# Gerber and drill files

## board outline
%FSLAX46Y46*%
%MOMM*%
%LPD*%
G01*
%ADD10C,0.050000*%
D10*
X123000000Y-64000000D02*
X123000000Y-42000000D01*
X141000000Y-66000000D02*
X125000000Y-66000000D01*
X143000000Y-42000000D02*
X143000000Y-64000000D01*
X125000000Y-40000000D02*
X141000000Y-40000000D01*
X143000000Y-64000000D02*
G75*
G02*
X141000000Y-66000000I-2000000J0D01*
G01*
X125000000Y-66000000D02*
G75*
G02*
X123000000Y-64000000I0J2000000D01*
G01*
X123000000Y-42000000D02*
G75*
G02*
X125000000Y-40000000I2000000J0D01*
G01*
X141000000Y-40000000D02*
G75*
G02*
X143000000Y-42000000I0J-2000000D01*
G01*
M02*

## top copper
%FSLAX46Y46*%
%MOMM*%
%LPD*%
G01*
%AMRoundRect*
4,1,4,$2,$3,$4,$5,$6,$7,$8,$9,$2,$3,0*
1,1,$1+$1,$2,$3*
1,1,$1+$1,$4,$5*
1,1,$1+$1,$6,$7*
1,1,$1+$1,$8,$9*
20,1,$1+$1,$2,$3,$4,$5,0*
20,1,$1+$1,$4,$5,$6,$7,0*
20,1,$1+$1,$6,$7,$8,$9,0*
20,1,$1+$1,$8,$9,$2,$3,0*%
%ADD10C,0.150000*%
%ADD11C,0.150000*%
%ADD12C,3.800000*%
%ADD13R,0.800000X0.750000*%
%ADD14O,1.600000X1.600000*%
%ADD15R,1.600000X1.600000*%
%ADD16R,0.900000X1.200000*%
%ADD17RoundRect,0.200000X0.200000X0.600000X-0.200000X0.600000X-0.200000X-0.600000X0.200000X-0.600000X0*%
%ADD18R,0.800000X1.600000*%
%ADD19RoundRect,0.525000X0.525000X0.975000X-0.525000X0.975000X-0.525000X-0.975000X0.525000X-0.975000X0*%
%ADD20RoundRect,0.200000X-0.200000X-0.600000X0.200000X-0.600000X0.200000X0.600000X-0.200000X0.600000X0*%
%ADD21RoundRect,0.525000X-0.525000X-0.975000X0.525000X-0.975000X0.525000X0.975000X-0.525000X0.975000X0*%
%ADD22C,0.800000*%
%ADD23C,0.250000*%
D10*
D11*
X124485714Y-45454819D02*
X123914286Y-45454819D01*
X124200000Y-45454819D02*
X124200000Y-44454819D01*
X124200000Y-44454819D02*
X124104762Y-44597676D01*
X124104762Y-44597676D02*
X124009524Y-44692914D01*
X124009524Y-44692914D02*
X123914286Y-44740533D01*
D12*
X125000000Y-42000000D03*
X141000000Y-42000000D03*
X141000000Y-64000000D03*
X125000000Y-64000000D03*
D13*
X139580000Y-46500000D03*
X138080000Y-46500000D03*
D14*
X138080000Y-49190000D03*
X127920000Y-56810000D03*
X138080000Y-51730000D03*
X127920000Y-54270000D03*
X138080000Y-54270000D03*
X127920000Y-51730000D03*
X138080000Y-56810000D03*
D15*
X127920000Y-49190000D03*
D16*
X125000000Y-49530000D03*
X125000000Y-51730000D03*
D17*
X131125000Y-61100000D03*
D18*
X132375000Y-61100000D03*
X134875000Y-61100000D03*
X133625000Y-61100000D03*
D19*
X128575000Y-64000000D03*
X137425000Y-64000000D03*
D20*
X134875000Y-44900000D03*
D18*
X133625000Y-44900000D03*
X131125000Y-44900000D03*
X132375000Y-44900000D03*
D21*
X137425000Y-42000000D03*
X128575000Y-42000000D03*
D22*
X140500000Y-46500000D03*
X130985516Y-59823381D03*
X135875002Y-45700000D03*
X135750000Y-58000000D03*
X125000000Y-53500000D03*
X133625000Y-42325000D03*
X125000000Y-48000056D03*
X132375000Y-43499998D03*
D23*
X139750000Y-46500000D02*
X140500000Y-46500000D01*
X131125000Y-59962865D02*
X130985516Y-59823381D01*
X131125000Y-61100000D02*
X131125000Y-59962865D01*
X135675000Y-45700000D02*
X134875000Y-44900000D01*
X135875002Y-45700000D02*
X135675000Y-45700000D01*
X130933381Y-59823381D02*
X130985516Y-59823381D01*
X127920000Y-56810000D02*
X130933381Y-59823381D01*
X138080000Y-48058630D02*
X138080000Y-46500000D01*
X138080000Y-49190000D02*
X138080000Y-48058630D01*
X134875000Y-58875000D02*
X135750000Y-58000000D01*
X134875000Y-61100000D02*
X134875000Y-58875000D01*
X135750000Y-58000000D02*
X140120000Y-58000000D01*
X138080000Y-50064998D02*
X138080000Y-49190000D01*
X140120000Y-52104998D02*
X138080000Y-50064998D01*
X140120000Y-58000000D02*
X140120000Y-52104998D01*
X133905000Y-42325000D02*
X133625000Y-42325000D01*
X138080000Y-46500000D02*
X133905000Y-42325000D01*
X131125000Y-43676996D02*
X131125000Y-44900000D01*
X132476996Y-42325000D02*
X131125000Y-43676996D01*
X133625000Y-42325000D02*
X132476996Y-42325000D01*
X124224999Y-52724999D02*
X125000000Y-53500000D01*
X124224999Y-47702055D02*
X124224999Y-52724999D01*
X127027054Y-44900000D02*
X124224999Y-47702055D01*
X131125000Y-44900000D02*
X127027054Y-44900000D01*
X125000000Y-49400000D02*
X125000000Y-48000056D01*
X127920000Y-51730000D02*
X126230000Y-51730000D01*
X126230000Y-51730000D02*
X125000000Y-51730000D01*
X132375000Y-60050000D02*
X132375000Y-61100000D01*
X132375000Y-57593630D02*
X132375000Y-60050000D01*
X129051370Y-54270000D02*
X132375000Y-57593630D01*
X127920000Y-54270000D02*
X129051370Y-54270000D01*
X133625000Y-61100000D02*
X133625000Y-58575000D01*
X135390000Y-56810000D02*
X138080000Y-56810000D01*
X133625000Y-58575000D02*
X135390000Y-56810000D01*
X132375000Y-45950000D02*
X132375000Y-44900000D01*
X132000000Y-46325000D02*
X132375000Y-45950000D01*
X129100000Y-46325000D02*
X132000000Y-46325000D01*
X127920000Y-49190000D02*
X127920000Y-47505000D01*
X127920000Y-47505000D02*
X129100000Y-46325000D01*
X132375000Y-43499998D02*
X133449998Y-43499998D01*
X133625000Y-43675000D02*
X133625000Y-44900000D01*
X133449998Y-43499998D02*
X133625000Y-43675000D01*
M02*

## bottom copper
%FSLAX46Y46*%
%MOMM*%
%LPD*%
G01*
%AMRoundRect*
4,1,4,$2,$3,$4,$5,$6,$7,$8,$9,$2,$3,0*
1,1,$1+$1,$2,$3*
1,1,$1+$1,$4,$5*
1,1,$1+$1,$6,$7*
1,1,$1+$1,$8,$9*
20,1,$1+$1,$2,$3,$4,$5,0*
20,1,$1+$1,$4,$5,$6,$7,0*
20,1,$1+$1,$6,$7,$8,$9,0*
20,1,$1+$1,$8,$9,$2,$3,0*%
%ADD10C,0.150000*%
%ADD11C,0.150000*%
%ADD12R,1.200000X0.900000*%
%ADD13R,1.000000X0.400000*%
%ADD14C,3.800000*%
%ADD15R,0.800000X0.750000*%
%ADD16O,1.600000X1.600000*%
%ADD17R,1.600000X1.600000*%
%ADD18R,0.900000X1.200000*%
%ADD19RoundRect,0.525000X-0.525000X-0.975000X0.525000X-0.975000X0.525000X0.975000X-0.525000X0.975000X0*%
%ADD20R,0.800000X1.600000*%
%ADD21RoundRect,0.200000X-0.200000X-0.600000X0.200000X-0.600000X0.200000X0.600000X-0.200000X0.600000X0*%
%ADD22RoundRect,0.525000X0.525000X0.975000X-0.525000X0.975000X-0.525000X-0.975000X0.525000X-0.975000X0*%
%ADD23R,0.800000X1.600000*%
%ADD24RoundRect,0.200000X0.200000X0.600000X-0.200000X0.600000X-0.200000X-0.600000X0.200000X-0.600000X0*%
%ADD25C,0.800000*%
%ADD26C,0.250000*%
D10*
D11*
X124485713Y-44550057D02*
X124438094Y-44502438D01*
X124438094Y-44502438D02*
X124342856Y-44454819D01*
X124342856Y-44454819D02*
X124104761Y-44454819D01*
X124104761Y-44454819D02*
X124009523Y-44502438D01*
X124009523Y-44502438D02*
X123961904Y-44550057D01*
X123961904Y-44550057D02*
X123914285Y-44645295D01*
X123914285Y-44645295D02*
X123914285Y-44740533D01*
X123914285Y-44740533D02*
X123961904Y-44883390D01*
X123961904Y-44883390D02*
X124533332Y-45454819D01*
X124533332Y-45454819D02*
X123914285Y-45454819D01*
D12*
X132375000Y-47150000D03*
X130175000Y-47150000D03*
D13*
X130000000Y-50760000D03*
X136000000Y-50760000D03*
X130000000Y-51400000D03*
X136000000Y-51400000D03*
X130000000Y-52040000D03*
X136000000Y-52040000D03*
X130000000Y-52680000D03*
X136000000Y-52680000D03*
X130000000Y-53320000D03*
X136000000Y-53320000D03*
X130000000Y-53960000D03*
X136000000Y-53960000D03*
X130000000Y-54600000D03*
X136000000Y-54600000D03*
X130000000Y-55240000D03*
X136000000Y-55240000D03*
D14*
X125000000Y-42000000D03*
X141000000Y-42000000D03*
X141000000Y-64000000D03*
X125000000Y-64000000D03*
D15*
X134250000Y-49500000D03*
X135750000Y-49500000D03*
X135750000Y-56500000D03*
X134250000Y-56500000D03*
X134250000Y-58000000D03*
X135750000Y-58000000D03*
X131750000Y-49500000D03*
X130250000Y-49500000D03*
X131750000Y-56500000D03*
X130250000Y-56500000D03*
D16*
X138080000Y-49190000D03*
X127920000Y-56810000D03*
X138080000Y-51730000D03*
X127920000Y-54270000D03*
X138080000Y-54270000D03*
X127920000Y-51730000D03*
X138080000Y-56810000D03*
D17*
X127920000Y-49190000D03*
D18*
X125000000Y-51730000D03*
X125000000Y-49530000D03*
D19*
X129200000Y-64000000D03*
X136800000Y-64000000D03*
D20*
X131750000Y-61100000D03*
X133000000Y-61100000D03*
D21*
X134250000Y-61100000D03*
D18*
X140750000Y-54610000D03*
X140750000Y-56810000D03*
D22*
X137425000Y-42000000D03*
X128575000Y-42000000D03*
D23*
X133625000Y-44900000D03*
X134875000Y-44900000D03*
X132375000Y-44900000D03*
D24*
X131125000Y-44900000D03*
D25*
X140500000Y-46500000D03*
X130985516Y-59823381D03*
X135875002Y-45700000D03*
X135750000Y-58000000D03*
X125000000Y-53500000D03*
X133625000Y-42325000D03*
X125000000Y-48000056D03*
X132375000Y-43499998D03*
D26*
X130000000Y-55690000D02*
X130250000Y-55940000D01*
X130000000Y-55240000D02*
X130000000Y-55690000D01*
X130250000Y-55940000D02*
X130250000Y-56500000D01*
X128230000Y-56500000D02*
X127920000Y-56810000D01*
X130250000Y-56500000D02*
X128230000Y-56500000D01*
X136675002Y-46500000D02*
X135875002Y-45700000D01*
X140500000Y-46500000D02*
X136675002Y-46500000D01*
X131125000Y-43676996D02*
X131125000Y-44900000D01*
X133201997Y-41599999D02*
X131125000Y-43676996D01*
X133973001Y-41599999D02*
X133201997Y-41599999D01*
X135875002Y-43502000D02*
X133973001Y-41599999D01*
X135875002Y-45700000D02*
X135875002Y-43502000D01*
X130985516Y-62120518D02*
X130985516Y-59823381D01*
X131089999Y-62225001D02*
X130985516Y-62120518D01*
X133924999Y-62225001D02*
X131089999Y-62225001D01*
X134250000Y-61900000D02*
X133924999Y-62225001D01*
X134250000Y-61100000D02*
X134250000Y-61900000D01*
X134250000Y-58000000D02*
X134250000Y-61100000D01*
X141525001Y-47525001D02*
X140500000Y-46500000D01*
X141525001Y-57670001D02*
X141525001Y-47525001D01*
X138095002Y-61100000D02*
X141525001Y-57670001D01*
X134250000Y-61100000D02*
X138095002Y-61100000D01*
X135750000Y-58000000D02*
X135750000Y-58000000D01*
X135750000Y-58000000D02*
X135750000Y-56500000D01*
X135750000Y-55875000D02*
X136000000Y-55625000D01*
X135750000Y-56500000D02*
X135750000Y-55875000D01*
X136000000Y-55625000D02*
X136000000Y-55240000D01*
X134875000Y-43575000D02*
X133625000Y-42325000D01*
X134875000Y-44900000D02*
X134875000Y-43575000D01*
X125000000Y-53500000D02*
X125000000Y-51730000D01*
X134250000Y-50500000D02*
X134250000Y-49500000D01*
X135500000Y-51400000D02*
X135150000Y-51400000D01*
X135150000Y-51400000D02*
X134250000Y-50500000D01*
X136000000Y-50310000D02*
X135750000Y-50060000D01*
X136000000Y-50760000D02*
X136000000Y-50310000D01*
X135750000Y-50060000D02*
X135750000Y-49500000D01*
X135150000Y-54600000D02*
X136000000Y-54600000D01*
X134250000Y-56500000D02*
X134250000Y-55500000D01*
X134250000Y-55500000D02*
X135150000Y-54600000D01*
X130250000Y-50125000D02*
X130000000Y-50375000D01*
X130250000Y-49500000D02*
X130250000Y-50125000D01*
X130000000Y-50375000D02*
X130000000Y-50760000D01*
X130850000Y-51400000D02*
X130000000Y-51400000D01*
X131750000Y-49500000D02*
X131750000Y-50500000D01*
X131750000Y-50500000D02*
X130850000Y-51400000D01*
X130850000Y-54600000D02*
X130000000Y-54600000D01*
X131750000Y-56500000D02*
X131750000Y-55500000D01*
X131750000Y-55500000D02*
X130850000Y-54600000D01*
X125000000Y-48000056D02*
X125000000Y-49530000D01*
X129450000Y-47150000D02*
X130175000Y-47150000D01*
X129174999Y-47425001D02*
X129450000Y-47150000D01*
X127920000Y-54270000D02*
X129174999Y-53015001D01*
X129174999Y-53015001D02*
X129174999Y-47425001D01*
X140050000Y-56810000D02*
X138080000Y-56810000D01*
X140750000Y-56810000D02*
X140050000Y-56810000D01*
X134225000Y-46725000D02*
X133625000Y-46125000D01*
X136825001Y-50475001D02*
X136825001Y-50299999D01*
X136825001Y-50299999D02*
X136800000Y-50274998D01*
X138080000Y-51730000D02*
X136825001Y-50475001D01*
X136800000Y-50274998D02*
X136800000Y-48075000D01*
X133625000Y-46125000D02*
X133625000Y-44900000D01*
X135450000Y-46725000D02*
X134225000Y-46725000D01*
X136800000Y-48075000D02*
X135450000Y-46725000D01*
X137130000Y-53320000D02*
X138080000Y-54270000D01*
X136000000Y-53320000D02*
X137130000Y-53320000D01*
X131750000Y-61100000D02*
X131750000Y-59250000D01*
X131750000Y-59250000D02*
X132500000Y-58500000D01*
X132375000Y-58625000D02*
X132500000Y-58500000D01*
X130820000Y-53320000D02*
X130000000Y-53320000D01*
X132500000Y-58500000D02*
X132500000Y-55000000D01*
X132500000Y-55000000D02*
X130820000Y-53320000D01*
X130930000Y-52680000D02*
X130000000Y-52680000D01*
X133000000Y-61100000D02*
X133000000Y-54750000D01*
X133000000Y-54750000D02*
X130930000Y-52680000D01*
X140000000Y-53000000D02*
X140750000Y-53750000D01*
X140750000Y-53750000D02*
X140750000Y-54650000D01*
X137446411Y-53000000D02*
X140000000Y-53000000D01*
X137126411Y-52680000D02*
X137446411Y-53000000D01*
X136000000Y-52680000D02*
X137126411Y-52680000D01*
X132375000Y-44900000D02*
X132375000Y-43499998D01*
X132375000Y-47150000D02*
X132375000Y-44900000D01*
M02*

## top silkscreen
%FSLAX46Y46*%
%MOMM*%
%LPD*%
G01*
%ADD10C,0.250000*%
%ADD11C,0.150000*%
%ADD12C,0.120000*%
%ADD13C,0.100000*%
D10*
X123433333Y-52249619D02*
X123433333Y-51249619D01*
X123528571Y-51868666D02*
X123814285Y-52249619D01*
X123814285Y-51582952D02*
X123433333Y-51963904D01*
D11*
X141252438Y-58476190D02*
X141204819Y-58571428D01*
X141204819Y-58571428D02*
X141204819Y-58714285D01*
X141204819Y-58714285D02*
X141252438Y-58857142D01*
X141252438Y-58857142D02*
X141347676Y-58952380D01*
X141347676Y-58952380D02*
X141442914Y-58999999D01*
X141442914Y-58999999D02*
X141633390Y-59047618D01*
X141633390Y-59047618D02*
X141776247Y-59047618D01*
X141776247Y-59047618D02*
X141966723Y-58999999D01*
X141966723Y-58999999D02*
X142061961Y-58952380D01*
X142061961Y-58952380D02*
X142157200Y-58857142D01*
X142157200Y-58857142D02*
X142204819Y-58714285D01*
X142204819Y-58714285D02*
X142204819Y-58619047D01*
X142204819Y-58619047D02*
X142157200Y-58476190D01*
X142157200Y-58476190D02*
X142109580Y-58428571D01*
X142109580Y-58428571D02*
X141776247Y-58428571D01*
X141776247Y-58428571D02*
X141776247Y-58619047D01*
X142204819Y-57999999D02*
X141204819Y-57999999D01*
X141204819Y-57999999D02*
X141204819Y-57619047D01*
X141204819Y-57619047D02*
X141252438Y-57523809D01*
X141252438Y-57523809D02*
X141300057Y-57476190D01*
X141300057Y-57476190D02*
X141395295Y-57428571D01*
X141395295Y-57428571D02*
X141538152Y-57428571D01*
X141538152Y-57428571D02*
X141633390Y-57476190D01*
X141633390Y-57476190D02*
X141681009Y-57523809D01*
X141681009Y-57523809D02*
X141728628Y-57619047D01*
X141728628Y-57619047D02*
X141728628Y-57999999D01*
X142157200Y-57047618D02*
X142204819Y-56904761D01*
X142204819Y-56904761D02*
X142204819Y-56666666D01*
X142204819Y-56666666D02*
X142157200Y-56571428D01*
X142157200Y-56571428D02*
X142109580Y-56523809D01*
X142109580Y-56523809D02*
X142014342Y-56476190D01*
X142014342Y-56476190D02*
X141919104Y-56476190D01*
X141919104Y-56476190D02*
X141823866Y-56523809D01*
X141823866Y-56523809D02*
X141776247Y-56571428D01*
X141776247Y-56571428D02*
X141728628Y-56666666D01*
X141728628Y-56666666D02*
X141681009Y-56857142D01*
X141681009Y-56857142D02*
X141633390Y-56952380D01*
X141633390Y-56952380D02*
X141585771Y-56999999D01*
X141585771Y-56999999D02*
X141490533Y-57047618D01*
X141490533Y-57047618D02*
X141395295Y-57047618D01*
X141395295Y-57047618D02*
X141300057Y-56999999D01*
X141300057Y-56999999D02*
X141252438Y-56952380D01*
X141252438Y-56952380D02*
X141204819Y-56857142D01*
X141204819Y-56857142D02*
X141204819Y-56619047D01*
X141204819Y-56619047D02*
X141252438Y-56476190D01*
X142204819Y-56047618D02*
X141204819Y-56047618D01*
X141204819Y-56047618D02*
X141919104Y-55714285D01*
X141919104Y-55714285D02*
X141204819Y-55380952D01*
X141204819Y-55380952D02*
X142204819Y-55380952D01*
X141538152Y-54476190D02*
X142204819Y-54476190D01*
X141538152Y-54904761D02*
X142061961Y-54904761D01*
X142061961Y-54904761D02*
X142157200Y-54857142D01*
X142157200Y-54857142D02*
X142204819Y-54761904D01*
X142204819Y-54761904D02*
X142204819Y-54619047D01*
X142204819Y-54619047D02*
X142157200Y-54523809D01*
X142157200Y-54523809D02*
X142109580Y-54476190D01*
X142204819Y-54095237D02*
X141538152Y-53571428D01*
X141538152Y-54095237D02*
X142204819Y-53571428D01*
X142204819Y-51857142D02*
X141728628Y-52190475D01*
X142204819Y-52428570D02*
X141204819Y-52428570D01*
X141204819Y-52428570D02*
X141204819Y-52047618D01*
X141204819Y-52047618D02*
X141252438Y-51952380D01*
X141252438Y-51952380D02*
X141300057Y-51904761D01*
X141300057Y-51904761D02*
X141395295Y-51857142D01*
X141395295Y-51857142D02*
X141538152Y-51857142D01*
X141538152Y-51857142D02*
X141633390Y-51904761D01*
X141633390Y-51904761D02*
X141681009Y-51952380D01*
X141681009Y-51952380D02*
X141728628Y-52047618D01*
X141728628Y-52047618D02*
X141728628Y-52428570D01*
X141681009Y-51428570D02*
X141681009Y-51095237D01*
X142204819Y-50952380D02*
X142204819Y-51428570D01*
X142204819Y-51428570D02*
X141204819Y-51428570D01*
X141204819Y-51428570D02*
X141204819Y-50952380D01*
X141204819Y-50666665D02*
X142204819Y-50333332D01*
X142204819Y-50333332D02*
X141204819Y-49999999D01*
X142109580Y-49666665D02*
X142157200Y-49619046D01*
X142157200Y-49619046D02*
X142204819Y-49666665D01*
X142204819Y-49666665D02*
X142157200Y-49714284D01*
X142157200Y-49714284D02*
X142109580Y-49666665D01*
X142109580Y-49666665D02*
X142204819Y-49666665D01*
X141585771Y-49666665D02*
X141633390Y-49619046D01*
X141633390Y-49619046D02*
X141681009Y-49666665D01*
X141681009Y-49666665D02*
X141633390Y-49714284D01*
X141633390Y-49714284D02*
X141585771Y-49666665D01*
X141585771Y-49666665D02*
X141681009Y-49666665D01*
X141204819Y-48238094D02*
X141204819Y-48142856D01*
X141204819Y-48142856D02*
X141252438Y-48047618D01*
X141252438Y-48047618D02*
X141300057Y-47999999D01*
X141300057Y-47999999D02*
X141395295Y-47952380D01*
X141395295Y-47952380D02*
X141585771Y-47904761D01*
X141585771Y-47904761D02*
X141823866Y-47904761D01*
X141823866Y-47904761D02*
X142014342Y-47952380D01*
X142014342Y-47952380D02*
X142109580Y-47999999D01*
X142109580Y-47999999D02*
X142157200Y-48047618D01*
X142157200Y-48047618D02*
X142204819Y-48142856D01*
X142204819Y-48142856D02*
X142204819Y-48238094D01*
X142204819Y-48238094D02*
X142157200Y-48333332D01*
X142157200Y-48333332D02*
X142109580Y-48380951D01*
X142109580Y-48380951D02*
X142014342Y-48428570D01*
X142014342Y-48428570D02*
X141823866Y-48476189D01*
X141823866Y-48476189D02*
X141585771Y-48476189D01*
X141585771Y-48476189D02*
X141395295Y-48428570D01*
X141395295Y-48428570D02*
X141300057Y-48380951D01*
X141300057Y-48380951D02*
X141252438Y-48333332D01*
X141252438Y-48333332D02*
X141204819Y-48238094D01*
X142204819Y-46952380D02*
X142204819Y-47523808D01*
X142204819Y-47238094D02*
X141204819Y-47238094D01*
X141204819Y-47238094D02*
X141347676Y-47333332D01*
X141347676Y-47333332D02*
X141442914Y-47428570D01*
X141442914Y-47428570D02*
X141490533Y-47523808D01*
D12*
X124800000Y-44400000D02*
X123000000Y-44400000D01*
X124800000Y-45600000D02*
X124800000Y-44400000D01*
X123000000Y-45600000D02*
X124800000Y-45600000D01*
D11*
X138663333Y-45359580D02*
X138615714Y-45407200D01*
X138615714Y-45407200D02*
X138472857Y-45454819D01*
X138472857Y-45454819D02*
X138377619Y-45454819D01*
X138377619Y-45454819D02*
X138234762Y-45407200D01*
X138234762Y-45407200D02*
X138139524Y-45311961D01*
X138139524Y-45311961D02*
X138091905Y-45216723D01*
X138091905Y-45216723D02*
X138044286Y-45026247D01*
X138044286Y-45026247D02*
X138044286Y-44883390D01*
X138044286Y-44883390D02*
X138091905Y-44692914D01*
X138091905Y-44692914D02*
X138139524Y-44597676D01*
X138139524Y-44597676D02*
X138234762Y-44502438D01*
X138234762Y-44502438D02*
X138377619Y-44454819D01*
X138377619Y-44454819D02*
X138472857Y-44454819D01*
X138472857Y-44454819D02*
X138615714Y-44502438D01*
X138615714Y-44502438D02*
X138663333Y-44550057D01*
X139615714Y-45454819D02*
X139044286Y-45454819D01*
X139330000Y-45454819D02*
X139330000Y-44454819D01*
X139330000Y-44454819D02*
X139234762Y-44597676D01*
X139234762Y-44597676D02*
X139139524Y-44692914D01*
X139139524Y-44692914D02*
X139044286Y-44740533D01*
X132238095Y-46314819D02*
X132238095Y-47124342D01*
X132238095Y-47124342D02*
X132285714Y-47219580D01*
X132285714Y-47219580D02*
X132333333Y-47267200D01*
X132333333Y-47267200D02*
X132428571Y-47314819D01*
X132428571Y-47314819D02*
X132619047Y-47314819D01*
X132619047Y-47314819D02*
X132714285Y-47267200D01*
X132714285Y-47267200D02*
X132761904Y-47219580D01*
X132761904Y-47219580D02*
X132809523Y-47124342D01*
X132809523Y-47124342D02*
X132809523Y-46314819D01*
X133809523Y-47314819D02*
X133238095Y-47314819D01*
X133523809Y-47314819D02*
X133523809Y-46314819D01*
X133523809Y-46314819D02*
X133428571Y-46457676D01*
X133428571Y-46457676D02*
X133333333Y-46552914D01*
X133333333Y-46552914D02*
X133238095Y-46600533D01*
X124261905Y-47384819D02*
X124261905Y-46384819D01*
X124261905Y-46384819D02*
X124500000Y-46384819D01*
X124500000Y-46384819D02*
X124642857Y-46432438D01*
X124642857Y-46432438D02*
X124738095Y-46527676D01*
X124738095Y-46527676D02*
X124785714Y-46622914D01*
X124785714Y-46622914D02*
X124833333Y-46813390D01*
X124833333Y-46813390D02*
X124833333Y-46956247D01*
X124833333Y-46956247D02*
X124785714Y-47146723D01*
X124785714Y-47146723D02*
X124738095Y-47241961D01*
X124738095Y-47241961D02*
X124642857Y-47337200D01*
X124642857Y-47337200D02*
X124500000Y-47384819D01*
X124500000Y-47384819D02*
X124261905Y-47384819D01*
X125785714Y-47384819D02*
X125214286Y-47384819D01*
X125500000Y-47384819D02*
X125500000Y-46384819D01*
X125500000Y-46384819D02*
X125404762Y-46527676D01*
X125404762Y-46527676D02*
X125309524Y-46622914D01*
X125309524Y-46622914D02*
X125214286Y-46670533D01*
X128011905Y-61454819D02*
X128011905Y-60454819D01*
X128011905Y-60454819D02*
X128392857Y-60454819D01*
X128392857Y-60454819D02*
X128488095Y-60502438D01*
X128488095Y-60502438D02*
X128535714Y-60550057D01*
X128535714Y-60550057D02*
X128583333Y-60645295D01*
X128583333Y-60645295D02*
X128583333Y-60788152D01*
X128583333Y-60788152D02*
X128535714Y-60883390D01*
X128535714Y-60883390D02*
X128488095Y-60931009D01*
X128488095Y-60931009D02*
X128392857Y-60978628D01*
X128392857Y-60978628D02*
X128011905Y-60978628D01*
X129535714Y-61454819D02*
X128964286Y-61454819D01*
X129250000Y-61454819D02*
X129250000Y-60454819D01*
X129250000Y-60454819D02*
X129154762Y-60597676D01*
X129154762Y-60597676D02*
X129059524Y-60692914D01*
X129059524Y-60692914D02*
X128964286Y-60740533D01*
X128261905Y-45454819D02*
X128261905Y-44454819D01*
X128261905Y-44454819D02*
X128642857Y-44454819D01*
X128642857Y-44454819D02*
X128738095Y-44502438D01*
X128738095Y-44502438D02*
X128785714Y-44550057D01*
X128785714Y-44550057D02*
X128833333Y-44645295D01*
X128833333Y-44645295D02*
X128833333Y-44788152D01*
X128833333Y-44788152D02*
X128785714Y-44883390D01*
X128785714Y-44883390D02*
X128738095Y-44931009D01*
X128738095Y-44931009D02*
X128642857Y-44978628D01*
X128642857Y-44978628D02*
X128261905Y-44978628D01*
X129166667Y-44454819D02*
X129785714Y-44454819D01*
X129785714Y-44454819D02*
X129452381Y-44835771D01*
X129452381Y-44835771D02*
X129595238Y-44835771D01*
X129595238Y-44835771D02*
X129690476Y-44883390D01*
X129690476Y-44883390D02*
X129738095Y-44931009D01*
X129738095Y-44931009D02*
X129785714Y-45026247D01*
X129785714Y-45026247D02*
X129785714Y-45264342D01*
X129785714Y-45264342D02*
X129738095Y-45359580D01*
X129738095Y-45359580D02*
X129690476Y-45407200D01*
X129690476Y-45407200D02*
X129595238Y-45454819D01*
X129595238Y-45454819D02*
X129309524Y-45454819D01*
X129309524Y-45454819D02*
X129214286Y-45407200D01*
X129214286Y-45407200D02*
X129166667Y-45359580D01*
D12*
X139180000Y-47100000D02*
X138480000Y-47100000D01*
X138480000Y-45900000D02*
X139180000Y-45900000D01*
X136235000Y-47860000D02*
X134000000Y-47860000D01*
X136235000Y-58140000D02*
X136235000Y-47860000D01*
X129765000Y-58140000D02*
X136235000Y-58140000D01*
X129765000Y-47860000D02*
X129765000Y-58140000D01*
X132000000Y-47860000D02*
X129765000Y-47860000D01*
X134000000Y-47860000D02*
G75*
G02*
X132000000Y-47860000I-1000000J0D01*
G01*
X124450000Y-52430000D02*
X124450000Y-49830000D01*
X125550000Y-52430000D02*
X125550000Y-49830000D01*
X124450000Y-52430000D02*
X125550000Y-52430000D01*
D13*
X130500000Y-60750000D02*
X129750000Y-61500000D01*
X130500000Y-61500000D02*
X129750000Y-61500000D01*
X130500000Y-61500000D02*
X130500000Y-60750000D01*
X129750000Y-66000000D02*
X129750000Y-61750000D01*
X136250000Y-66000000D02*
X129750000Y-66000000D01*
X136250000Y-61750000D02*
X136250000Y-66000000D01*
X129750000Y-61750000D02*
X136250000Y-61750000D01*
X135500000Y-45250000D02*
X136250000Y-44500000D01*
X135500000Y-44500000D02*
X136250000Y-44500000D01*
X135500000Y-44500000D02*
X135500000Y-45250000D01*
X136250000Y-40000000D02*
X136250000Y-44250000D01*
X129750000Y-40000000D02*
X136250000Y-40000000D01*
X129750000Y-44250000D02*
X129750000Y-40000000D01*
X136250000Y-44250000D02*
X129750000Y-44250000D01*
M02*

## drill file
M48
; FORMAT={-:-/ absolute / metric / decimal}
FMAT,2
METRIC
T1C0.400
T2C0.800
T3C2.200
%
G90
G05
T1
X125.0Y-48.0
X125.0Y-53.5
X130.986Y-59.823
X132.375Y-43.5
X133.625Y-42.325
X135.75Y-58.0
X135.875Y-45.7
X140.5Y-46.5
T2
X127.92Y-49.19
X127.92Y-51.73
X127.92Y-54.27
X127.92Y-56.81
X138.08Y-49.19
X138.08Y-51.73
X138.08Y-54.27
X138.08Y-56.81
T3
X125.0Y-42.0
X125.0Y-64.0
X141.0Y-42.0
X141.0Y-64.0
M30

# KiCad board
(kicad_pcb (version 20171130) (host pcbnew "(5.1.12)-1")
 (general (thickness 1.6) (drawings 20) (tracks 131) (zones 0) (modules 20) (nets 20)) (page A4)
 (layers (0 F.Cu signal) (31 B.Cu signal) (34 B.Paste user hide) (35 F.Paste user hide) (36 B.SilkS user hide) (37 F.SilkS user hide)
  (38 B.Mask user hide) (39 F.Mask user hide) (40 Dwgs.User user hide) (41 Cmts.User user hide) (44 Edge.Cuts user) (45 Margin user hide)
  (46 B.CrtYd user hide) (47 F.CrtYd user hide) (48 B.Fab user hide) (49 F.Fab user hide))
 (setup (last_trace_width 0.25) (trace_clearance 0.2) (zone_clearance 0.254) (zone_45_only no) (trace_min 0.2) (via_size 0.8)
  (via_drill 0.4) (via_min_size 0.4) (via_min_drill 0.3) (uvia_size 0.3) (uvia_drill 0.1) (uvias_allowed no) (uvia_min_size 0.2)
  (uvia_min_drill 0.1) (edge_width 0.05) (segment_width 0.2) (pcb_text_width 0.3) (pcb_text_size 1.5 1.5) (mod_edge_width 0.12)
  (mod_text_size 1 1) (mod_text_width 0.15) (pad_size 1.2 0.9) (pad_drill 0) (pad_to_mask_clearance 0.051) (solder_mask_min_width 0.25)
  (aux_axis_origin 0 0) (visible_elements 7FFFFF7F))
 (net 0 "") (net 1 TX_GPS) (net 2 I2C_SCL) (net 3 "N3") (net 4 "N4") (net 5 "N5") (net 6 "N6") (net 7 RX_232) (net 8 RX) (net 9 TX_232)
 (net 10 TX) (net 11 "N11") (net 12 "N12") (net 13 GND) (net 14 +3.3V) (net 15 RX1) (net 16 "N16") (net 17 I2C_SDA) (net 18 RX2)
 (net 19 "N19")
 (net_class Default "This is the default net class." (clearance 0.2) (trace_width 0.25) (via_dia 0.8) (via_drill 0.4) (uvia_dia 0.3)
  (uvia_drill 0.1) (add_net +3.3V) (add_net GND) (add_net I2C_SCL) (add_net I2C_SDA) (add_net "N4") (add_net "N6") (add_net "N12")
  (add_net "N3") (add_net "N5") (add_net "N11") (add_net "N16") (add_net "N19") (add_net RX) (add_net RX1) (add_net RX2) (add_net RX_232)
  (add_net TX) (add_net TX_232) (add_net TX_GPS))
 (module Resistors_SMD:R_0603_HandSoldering (layer B.Cu) (at 131.275 47.15 180)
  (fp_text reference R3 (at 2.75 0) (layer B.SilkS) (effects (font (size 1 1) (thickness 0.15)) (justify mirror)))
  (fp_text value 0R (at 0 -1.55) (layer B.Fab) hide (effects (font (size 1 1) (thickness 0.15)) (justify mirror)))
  (pad 1 smd rect (at -1.1 0 180) (size 1.2 0.9) (layers B.Cu B.Paste B.Mask) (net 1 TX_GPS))
  (pad 2 smd rect (at 1.1 0 180) (size 1.2 0.9) (layers B.Cu B.Paste B.Mask) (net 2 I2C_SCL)))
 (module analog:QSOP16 (layer B.Cu) (at 133 53 270) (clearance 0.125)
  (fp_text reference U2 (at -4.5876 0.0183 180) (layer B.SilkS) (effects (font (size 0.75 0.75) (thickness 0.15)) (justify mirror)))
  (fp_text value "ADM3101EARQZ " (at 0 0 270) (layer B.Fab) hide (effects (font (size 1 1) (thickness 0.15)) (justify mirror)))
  (pad 16 smd rect (at -2.24 3 270) (size 0.4 1) (layers B.Cu B.Paste B.Mask) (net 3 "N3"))
  (pad 1 smd rect (at -2.24 -3 270) (size 0.4 1) (layers B.Cu B.Paste B.Mask) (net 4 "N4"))
  (pad 15 smd rect (at -1.6 3 270) (size 0.4 1) (layers B.Cu B.Paste B.Mask) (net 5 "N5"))
  (pad 2 smd rect (at -1.6 -3 270) (size 0.4 1) (layers B.Cu B.Paste B.Mask) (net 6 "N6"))
  (pad 14 smd rect (at -0.96 3 270) (size 0.4 1) (layers B.Cu B.Paste B.Mask))
  (pad 3 smd rect (at -0.96 -3 270) (size 0.4 1) (layers B.Cu B.Paste B.Mask))
  (pad 13 smd rect (at -0.32 3 270) (size 0.4 1) (layers B.Cu B.Paste B.Mask) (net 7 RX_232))
  (pad 4 smd rect (at -0.32 -3 270) (size 0.4 1) (layers B.Cu B.Paste B.Mask) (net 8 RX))
  (pad 12 smd rect (at 0.32 3 270) (size 0.4 1) (layers B.Cu B.Paste B.Mask) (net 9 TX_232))
  (pad 5 smd rect (at 0.32 -3 270) (size 0.4 1) (layers B.Cu B.Paste B.Mask) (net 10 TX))
  (pad 11 smd rect (at 0.96 3 270) (size 0.4 1) (layers B.Cu B.Paste B.Mask))
  (pad 6 smd rect (at 0.96 -3 270) (size 0.4 1) (layers B.Cu B.Paste B.Mask))
  (pad 10 smd rect (at 1.6 3 270) (size 0.4 1) (layers B.Cu B.Paste B.Mask) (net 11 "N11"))
  (pad 7 smd rect (at 1.6 -3 270) (size 0.4 1) (layers B.Cu B.Paste B.Mask) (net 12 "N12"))
  (pad 9 smd rect (at 2.24 3 270) (size 0.4 1) (layers B.Cu B.Paste B.Mask) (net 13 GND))
  (pad 8 smd rect (at 2.24 -3 270) (size 0.4 1) (layers B.Cu B.Paste B.Mask) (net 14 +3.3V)))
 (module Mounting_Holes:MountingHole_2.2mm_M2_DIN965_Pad (layer F.Cu) (at 125 42)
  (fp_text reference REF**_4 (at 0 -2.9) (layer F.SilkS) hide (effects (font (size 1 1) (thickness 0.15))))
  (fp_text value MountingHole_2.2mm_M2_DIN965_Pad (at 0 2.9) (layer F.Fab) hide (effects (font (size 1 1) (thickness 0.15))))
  (pad 1 thru_hole circle (at 0 0) (size 3.8 3.8) (drill 2.2) (layers *.Cu *.Mask)))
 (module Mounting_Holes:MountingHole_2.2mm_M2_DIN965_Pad (layer F.Cu) (at 141 42)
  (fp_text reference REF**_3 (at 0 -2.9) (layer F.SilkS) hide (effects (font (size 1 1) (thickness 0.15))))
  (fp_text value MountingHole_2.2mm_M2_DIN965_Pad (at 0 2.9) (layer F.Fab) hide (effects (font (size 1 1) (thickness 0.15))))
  (pad 1 thru_hole circle (at 0 0) (size 3.8 3.8) (drill 2.2) (layers *.Cu *.Mask)))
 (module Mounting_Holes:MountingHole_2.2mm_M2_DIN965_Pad (layer F.Cu) (at 141 64)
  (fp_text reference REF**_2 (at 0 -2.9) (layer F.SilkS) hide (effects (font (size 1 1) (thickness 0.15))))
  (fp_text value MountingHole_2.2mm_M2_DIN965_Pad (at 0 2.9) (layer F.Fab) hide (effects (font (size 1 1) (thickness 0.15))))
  (pad 1 thru_hole circle (at 0 0) (size 3.8 3.8) (drill 2.2) (layers *.Cu *.Mask)))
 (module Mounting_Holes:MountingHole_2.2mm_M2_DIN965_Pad (layer F.Cu) (at 125 64)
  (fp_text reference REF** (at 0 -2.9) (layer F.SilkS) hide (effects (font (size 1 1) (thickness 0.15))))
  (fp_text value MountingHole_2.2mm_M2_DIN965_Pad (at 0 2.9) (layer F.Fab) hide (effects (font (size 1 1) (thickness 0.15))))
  (pad 1 thru_hole circle (at 0 0) (size 3.8 3.8) (drill 2.2) (layers *.Cu *.Mask)))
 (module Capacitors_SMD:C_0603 (layer F.Cu) (at 138.83 46.5)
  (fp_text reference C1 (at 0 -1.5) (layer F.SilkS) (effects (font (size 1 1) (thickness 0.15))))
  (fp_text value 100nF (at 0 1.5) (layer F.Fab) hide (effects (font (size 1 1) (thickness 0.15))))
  (fp_line (start 0.35 0.6) (end -0.35 0.6) (layer F.SilkS) (width 0.12))
  (fp_line (start -0.35 -0.6) (end 0.35 -0.6) (layer F.SilkS) (width 0.12))
  (pad 2 smd rect (at 0.75 0) (size 0.8 0.75) (layers F.Cu F.Paste F.Mask) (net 13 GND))
  (pad 1 smd rect (at -0.75 0) (size 0.8 0.75) (layers F.Cu F.Paste F.Mask) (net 14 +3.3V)))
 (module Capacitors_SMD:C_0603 (layer B.Cu) (at 135 49.5 180)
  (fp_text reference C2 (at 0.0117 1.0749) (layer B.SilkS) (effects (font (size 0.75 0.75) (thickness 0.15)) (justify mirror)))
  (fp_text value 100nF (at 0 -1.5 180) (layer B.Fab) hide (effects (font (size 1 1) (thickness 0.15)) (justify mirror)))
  (pad 2 smd rect (at 0.75 0 180) (size 0.8 0.75) (layers B.Cu B.Paste B.Mask) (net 6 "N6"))
  (pad 1 smd rect (at -0.75 0 180) (size 0.8 0.75) (layers B.Cu B.Paste B.Mask) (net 4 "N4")))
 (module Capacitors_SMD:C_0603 (layer B.Cu) (at 135 56.5)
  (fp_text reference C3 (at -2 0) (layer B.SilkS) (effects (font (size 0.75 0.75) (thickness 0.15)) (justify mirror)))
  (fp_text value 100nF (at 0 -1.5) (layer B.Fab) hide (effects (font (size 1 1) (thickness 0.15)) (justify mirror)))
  (pad 2 smd rect (at 0.75 0) (size 0.8 0.75) (layers B.Cu B.Paste B.Mask) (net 14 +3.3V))
  (pad 1 smd rect (at -0.75 0) (size 0.8 0.75) (layers B.Cu B.Paste B.Mask) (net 12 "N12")))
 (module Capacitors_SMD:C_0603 (layer B.Cu) (at 135 58 180)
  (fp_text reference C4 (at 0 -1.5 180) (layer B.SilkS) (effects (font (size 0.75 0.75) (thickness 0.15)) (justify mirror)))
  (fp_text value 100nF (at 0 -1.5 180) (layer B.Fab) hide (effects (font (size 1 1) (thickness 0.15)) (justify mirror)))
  (pad 2 smd rect (at 0.75 0 180) (size 0.8 0.75) (layers B.Cu B.Paste B.Mask) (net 13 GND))
  (pad 1 smd rect (at -0.75 0 180) (size 0.8 0.75) (layers B.Cu B.Paste B.Mask) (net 14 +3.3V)))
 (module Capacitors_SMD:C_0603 (layer B.Cu) (at 131 49.5)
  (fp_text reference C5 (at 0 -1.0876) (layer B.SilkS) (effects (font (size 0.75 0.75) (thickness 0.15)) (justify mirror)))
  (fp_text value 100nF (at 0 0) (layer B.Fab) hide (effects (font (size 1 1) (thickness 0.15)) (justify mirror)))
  (pad 2 smd rect (at 0.75 0) (size 0.8 0.75) (layers B.Cu B.Paste B.Mask) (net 5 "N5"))
  (pad 1 smd rect (at -0.75 0) (size 0.8 0.75) (layers B.Cu B.Paste B.Mask) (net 3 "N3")))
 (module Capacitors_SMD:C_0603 (layer B.Cu) (at 131 56.5)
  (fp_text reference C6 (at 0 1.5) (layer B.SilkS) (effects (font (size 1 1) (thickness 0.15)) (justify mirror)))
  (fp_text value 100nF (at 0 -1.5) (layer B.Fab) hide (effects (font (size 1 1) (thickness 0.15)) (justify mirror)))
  (pad 2 smd rect (at 0.75 0) (size 0.8 0.75) (layers B.Cu B.Paste B.Mask) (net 11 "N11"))
  (pad 1 smd rect (at -0.75 0) (size 0.8 0.75) (layers B.Cu B.Paste B.Mask) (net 13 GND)))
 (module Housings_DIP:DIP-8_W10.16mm (layer F.Cu) (at 133 53)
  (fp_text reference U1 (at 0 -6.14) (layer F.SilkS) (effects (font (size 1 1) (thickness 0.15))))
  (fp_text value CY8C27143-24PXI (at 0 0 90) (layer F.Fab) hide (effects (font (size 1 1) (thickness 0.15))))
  (fp_line (start 3.235 -5.14) (end 1 -5.14) (layer F.SilkS) (width 0.12))
  (fp_line (start 3.235 5.14) (end 3.235 -5.14) (layer F.SilkS) (width 0.12))
  (fp_line (start -3.235 5.14) (end 3.235 5.14) (layer F.SilkS) (width 0.12))
  (fp_line (start -3.235 -5.14) (end -3.235 5.14) (layer F.SilkS) (width 0.12))
  (fp_line (start -1 -5.14) (end -3.235 -5.14) (layer F.SilkS) (width 0.12))
  (fp_arc (start 0 -5.14) (end -1 -5.14) (angle -180) (layer F.SilkS) (width 0.12))
  (pad 8 thru_hole oval (at 5.08 -3.81) (size 1.6 1.6) (drill 0.8) (layers *.Cu *.Mask) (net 14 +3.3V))
  (pad 4 thru_hole oval (at -5.08 3.81) (size 1.6 1.6) (drill 0.8) (layers *.Cu *.Mask) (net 13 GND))
  (pad 7 thru_hole oval (at 5.08 -1.27) (size 1.6 1.6) (drill 0.8) (layers *.Cu *.Mask) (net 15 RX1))
  (pad 3 thru_hole oval (at -5.08 1.27) (size 1.6 1.6) (drill 0.8) (layers *.Cu *.Mask) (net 2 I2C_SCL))
  (pad 6 thru_hole oval (at 5.08 1.27) (size 1.6 1.6) (drill 0.8) (layers *.Cu *.Mask) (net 10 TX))
  (pad 2 thru_hole oval (at -5.08 -1.27) (size 1.6 1.6) (drill 0.8) (layers *.Cu *.Mask) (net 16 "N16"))
  (pad 5 thru_hole oval (at 5.08 3.81) (size 1.6 1.6) (drill 0.8) (layers *.Cu *.Mask) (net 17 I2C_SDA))
  (pad 1 thru_hole rect (at -5.08 -3.81) (size 1.6 1.6) (drill 0.8) (layers *.Cu *.Mask) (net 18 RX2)))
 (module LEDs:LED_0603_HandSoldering (layer F.Cu) (at 125 50.63 90)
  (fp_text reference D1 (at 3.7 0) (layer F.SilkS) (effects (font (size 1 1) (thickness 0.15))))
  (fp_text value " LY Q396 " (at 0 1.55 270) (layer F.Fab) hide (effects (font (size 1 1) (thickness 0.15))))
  (fp_line (start -1.8 -0.55) (end 0.8 -0.55) (layer F.SilkS) (width 0.12))
  (fp_line (start -1.8 0.55) (end 0.8 0.55) (layer F.SilkS) (width 0.12))
  (fp_line (start -1.8 -0.55) (end -1.8 0.55) (layer F.SilkS) (width 0.12))
  (pad 2 smd rect (at 1.1 0 90) (size 1.2 0.9) (layers F.Cu F.Paste F.Mask) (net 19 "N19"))
  (pad 1 smd rect (at -1.1 0 90) (size 1.2 0.9) (layers F.Cu F.Paste F.Mask) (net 16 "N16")))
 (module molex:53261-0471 (layer F.Cu) (at 133 64 180) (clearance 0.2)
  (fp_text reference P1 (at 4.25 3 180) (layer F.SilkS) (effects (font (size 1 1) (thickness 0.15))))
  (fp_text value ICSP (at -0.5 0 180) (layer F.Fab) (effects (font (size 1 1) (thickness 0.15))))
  (fp_line (start 2.5 3.25) (end 3.25 2.5) (layer F.SilkS) (width 0.1))
  (fp_line (start 2.5 2.5) (end 3.25 2.5) (layer F.SilkS) (width 0.1))
  (fp_line (start 2.5 2.5) (end 2.5 3.25) (layer F.SilkS) (width 0.1))
  (fp_line (start 3.25 -2) (end 3.25 2.25) (layer F.SilkS) (width 0.1))
  (fp_line (start -3.25 -2) (end 3.25 -2) (layer F.SilkS) (width 0.1))
  (fp_line (start -3.25 2.25) (end -3.25 -2) (layer F.SilkS) (width 0.1))
  (fp_line (start 3.25 2.25) (end -3.25 2.25) (layer F.SilkS) (width 0.1))
  (pad 1 connect roundrect (at 1.875 2.9 180) (size 0.8 1.6) (layers F.Cu F.Mask) (roundrect_rratio 0.25) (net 13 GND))
  (pad 2 connect rect (at 0.625 2.9 180) (size 0.8 1.6) (layers F.Cu F.Mask) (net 2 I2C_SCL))
  (pad 4 connect rect (at -1.875 2.9 180) (size 0.8 1.6) (layers F.Cu F.Mask) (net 14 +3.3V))
  (pad 3 connect rect (at -0.625 2.9 180) (size 0.8 1.6) (layers F.Cu F.Mask) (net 17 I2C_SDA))
  (pad "" connect roundrect (at 4.425 0 180) (size 2.1 3) (layers F.Cu F.Mask) (roundrect_rratio 0.25))
  (pad "" connect roundrect (at -4.425 0 180) (size 2.1 3) (layers F.Cu F.Mask) (roundrect_rratio 0.25)))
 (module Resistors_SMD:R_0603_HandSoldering (layer B.Cu) (at 125 50.63 270)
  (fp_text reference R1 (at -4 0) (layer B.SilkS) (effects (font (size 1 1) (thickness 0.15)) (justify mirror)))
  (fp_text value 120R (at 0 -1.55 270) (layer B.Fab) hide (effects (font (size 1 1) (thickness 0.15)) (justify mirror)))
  (pad 2 smd rect (at 1.1 0 270) (size 1.2 0.9) (layers B.Cu B.Paste B.Mask) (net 14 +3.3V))
  (pad 1 smd rect (at -1.1 0 270) (size 1.2 0.9) (layers B.Cu B.Paste B.Mask) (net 19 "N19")))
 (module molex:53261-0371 (layer B.Cu) (at 133 64) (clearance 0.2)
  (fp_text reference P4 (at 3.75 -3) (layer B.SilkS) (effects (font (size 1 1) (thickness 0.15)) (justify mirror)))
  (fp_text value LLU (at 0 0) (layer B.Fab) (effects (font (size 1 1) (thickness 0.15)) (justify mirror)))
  (pad "" connect roundrect (at -3.8 0) (size 2.1 3) (layers B.Cu B.Mask) (roundrect_rratio 0.25))
  (pad "" connect roundrect (at 3.8 0) (size 2.1 3) (layers B.Cu B.Mask) (roundrect_rratio 0.25))
  (pad 3 smd rect (at -1.25 -2.9) (size 0.8 1.6) (layers B.Cu B.Paste B.Mask) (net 9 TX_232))
  (pad 2 smd rect (at 0 -2.9) (size 0.8 1.6) (layers B.Cu B.Paste B.Mask) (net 7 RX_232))
  (pad 1 smd roundrect (at 1.25 -2.9) (size 0.8 1.6) (layers B.Cu B.Paste B.Mask) (roundrect_rratio 0.25) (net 13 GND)))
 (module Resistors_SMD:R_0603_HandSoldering (layer B.Cu) (at 140.75 55.71 90)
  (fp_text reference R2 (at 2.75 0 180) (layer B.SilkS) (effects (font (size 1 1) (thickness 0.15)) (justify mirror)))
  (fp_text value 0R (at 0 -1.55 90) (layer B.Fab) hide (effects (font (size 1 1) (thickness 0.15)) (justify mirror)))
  (pad 2 smd rect (at 1.1 0 90) (size 1.2 0.9) (layers B.Cu B.Paste B.Mask) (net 8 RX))
  (pad 1 smd rect (at -1.1 0 90) (size 1.2 0.9) (layers B.Cu B.Paste B.Mask) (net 17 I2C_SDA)))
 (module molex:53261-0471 (layer B.Cu) (at 133 42 180) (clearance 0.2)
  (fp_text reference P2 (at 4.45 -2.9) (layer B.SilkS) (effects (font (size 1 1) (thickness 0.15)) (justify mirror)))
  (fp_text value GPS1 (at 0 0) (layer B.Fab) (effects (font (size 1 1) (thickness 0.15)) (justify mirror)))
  (pad "" connect roundrect (at -4.425 0 180) (size 2.1 3) (layers B.Cu B.Mask) (roundrect_rratio 0.25))
  (pad "" connect roundrect (at 4.425 0 180) (size 2.1 3) (layers B.Cu B.Mask) (roundrect_rratio 0.25))
  (pad 3 connect rect (at -0.625 -2.9 180) (size 0.8 1.6) (layers B.Cu B.Mask) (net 15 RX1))
  (pad 4 connect rect (at -1.875 -2.9 180) (size 0.8 1.6) (layers B.Cu B.Mask) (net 14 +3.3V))
  (pad 2 connect rect (at 0.625 -2.9 180) (size 0.8 1.6) (layers B.Cu B.Mask) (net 1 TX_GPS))
  (pad 1 connect roundrect (at 1.875 -2.9 180) (size 0.8 1.6) (layers B.Cu B.Mask) (roundrect_rratio 0.25) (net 13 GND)))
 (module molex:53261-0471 (layer F.Cu) (at 133 42) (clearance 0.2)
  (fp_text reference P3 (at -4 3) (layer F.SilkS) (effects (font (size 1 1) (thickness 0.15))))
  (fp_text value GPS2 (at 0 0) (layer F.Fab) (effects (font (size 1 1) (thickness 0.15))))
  (fp_line (start 2.5 3.25) (end 3.25 2.5) (layer F.SilkS) (width 0.1))
  (fp_line (start 2.5 2.5) (end 3.25 2.5) (layer F.SilkS) (width 0.1))
  (fp_line (start 2.5 2.5) (end 2.5 3.25) (layer F.SilkS) (width 0.1))
  (fp_line (start 3.25 -2) (end 3.25 2.25) (layer F.SilkS) (width 0.1))
  (fp_line (start -3.25 -2) (end 3.25 -2) (layer F.SilkS) (width 0.1))
  (fp_line (start -3.25 2.25) (end -3.25 -2) (layer F.SilkS) (width 0.1))
  (fp_line (start 3.25 2.25) (end -3.25 2.25) (layer F.SilkS) (width 0.1))
  (pad 1 connect roundrect (at 1.875 2.9) (size 0.8 1.6) (layers F.Cu F.Mask) (roundrect_rratio 0.25) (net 13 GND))
  (pad 2 connect rect (at 0.625 2.9) (size 0.8 1.6) (layers F.Cu F.Mask) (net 1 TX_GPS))
  (pad 4 connect rect (at -1.875 2.9) (size 0.8 1.6) (layers F.Cu F.Mask) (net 14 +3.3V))
  (pad 3 connect rect (at -0.625 2.9) (size 0.8 1.6) (layers F.Cu F.Mask) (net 18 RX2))
  (pad "" connect roundrect (at 4.425 0) (size 2.1 3) (layers F.Cu F.Mask) (roundrect_rratio 0.25))
  (pad "" connect roundrect (at -4.425 0) (size 2.1 3) (layers F.Cu F.Mask) (roundrect_rratio 0.25)))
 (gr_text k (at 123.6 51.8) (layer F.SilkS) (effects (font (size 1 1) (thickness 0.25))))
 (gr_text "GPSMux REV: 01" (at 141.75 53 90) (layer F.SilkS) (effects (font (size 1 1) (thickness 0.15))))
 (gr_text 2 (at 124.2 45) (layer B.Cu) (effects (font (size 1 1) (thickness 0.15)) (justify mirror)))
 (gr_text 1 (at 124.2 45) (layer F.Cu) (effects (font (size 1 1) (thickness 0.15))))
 (gr_line (start 124.8 44.4) (end 123 44.4) (layer F.SilkS) (width 0.12))
 (gr_line (start 124.8 45.6) (end 124.8 44.4) (layer F.SilkS) (width 0.12))
 (gr_line (start 123 45.6) (end 124.8 45.6) (layer F.SilkS) (width 0.12))
 (gr_line (start 123 64) (end 123 42) (layer Edge.Cuts) (width 0.05))
 (gr_line (start 141 66) (end 125 66) (layer Edge.Cuts) (width 0.05))
 (gr_line (start 143 42) (end 143 64) (layer Edge.Cuts) (width 0.05))
 (gr_line (start 125 40) (end 141 40) (layer Edge.Cuts) (width 0.05))
 (gr_arc (start 141 64) (end 141 66) (angle -90) (layer Edge.Cuts) (width 0.05))
 (gr_arc (start 125 64) (end 123 64) (angle -90) (layer Edge.Cuts) (width 0.05))
 (gr_arc (start 125 42) (end 125 40) (angle -90) (layer Edge.Cuts) (width 0.05))
 (gr_arc (start 141 42) (end 143 42) (angle -90) (layer Edge.Cuts) (width 0.05))
 (via (at 140.5 46.5) (size 0.8) (drill 0.4) (layers F.Cu B.Cu) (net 13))
 (via (at 130.985516 59.823381) (size 0.8) (drill 0.4) (layers F.Cu B.Cu) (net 13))
 (via (at 135.875002 45.7) (size 0.8) (drill 0.4) (layers F.Cu B.Cu) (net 13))
 (via (at 135.75 58) (size 0.8) (drill 0.4) (layers F.Cu B.Cu) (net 14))
 (via (at 125 53.5) (size 0.8) (drill 0.4) (layers F.Cu B.Cu) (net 14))
 (via (at 133.625 42.325) (size 0.8) (drill 0.4) (layers F.Cu B.Cu) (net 14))
 (via (at 125 48.000056) (size 0.8) (drill 0.4) (layers F.Cu B.Cu) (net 19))
 (via (at 132.375 43.499998) (size 0.8) (drill 0.4) (layers F.Cu B.Cu) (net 1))
 (segment (start 139.75 46.5) (end 140.5 46.5) (width 0.25) (layer F.Cu) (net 13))
 (segment (start 131.125 59.962865) (end 130.985516 59.823381) (width 0.25) (layer F.Cu) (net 13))
 (segment (start 131.125 61.1) (end 131.125 59.962865) (width 0.25) (layer F.Cu) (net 13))
 (segment (start 130 55.69) (end 130.25 55.94) (width 0.25) (layer B.Cu) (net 13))
 (segment (start 130 55.24) (end 130 55.69) (width 0.25) (layer B.Cu) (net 13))
 (segment (start 130.25 55.94) (end 130.25 56.5) (width 0.25) (layer B.Cu) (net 13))
 (segment (start 135.675 45.7) (end 134.875 44.9) (width 0.25) (layer F.Cu) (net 13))
 (segment (start 135.875002 45.7) (end 135.675 45.7) (width 0.25) (layer F.Cu) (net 13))
 (segment (start 130.933381 59.823381) (end 130.985516 59.823381) (width 0.25) (layer F.Cu) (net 13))
 (segment (start 127.92 56.81) (end 130.933381 59.823381) (width 0.25) (layer F.Cu) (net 13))
 (segment (start 128.23 56.5) (end 127.92 56.81) (width 0.25) (layer B.Cu) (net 13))
 (segment (start 130.25 56.5) (end 128.23 56.5) (width 0.25) (layer B.Cu) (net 13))
 (segment (start 136.675002 46.5) (end 135.875002 45.7) (width 0.25) (layer B.Cu) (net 13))
 (segment (start 140.5 46.5) (end 136.675002 46.5) (width 0.25) (layer B.Cu) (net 13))
 (segment (start 131.125 43.676996) (end 131.125 44.9) (width 0.25) (layer B.Cu) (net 13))
 (segment (start 133.201997 41.599999) (end 131.125 43.676996) (width 0.25) (layer B.Cu) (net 13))
 (segment (start 133.973001 41.599999) (end 133.201997 41.599999) (width 0.25) (layer B.Cu) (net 13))
 (segment (start 135.875002 43.502) (end 133.973001 41.599999) (width 0.25) (layer B.Cu) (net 13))
 (segment (start 135.875002 45.7) (end 135.875002 43.502) (width 0.25) (layer B.Cu) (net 13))
 (segment (start 130.985516 62.120518) (end 130.985516 59.823381) (width 0.25) (layer B.Cu) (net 13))
 (segment (start 131.089999 62.225001) (end 130.985516 62.120518) (width 0.25) (layer B.Cu) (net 13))
 (segment (start 133.924999 62.225001) (end 131.089999 62.225001) (width 0.25) (layer B.Cu) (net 13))
 (segment (start 134.25 61.9) (end 133.924999 62.225001) (width 0.25) (layer B.Cu) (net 13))
 (segment (start 134.25 61.1) (end 134.25 61.9) (width 0.25) (layer B.Cu) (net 13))
 (segment (start 134.25 58) (end 134.25 61.1) (width 0.25) (layer B.Cu) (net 13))
 (segment (start 141.525001 47.525001) (end 140.5 46.5) (width 0.25) (layer B.Cu) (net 13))
 (segment (start 141.525001 57.670001) (end 141.525001 47.525001) (width 0.25) (layer B.Cu) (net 13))
 (segment (start 138.095002 61.1) (end 141.525001 57.670001) (width 0.25) (layer B.Cu) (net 13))
 (segment (start 134.25 61.1) (end 138.095002 61.1) (width 0.25) (layer B.Cu) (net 13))
 (segment (start 135.75 58) (end 135.75 58) (width 0.25) (layer B.Cu) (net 14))
 (segment (start 138.08 48.05863) (end 138.08 46.5) (width 0.25) (layer F.Cu) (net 14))
 (segment (start 138.08 49.19) (end 138.08 48.05863) (width 0.25) (layer F.Cu) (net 14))
 (segment (start 135.75 58) (end 135.75 56.5) (width 0.25) (layer B.Cu) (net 14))
 (segment (start 135.75 55.875) (end 136 55.625) (width 0.25) (layer B.Cu) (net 14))
 (segment (start 135.75 56.5) (end 135.75 55.875) (width 0.25) (layer B.Cu) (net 14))
 (segment (start 136 55.625) (end 136 55.24) (width 0.25) (layer B.Cu) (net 14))
 (segment (start 134.875 43.575) (end 133.625 42.325) (width 0.25) (layer B.Cu) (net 14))
 (segment (start 134.875 44.9) (end 134.875 43.575) (width 0.25) (layer B.Cu) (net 14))
 (segment (start 125 53.5) (end 125 51.73) (width 0.25) (layer B.Cu) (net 14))
 (segment (start 134.875 58.875) (end 135.75 58) (width 0.25) (layer F.Cu) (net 14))
 (segment (start 134.875 61.1) (end 134.875 58.875) (width 0.25) (layer F.Cu) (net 14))
 (segment (start 135.75 58) (end 140.12 58) (width 0.25) (layer F.Cu) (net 14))
 (segment (start 138.08 50.064998) (end 138.08 49.19) (width 0.25) (layer F.Cu) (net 14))
 (segment (start 140.12 52.104998) (end 138.08 50.064998) (width 0.25) (layer F.Cu) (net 14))
 (segment (start 140.12 58) (end 140.12 52.104998) (width 0.25) (layer F.Cu) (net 14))
 (segment (start 133.905 42.325) (end 133.625 42.325) (width 0.25) (layer F.Cu) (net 14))
 (segment (start 138.08 46.5) (end 133.905 42.325) (width 0.25) (layer F.Cu) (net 14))
 (segment (start 131.125 43.676996) (end 131.125 44.9) (width 0.25) (layer F.Cu) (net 14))
 (segment (start 132.476996 42.325) (end 131.125 43.676996) (width 0.25) (layer F.Cu) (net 14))
 (segment (start 133.625 42.325) (end 132.476996 42.325) (width 0.25) (layer F.Cu) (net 14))
 (segment (start 124.224999 52.724999) (end 125 53.5) (width 0.25) (layer F.Cu) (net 14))
 (segment (start 124.224999 47.702055) (end 124.224999 52.724999) (width 0.25) (layer F.Cu) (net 14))
 (segment (start 127.027054 44.9) (end 124.224999 47.702055) (width 0.25) (layer F.Cu) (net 14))
 (segment (start 131.125 44.9) (end 127.027054 44.9) (width 0.25) (layer F.Cu) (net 14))
 (segment (start 134.25 50.5) (end 134.25 49.5) (width 0.25) (layer B.Cu) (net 6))
 (segment (start 135.5 51.4) (end 135.15 51.4) (width 0.25) (layer B.Cu) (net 6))
 (segment (start 135.15 51.4) (end 134.25 50.5) (width 0.25) (layer B.Cu) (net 6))
 (segment (start 136 50.31) (end 135.75 50.06) (width 0.25) (layer B.Cu) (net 4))
 (segment (start 136 50.76) (end 136 50.31) (width 0.25) (layer B.Cu) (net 4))
 (segment (start 135.75 50.06) (end 135.75 49.5) (width 0.25) (layer B.Cu) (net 4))
 (segment (start 135.15 54.6) (end 136 54.6) (width 0.25) (layer B.Cu) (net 12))
 (segment (start 134.25 56.5) (end 134.25 55.5) (width 0.25) (layer B.Cu) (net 12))
 (segment (start 134.25 55.5) (end 135.15 54.6) (width 0.25) (layer B.Cu) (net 12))
 (segment (start 130.25 50.125) (end 130 50.375) (width 0.25) (layer B.Cu) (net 3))
 (segment (start 130.25 49.5) (end 130.25 50.125) (width 0.25) (layer B.Cu) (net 3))
 (segment (start 130 50.375) (end 130 50.76) (width 0.25) (layer B.Cu) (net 3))
 (segment (start 130.85 51.4) (end 130 51.4) (width 0.25) (layer B.Cu) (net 5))
 (segment (start 131.75 49.5) (end 131.75 50.5) (width 0.25) (layer B.Cu) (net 5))
 (segment (start 131.75 50.5) (end 130.85 51.4) (width 0.25) (layer B.Cu) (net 5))
 (segment (start 130.85 54.6) (end 130 54.6) (width 0.25) (layer B.Cu) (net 11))
 (segment (start 131.75 56.5) (end 131.75 55.5) (width 0.25) (layer B.Cu) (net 11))
 (segment (start 131.75 55.5) (end 130.85 54.6) (width 0.25) (layer B.Cu) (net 11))
 (segment (start 125 49.4) (end 125 48.000056) (width 0.25) (layer F.Cu) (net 19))
 (segment (start 125 48.000056) (end 125 49.53) (width 0.25) (layer B.Cu) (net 19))
 (segment (start 127.92 51.73) (end 126.23 51.73) (width 0.25) (layer F.Cu) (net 16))
 (segment (start 126.23 51.73) (end 125 51.73) (width 0.25) (layer F.Cu) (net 16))
 (segment (start 132.375 60.05) (end 132.375 61.1) (width 0.25) (layer F.Cu) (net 2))
 (segment (start 132.375 57.59363) (end 132.375 60.05) (width 0.25) (layer F.Cu) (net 2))
 (segment (start 129.05137 54.27) (end 132.375 57.59363) (width 0.25) (layer F.Cu) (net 2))
 (segment (start 127.92 54.27) (end 129.05137 54.27) (width 0.25) (layer F.Cu) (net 2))
 (segment (start 129.45 47.15) (end 130.175 47.15) (width 0.25) (layer B.Cu) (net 2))
 (segment (start 129.174999 47.425001) (end 129.45 47.15) (width 0.25) (layer B.Cu) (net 2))
 (segment (start 127.92 54.27) (end 129.174999 53.015001) (width 0.25) (layer B.Cu) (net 2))
 (segment (start 129.174999 53.015001) (end 129.174999 47.425001) (width 0.25) (layer B.Cu) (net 2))
 (segment (start 140.05 56.81) (end 138.08 56.81) (width 0.25) (layer B.Cu) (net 17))
 (segment (start 140.75 56.81) (end 140.05 56.81) (width 0.25) (layer B.Cu) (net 17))
 (segment (start 133.625 61.1) (end 133.625 58.575) (width 0.25) (layer F.Cu) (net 17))
 (segment (start 135.39 56.81) (end 138.08 56.81) (width 0.25) (layer F.Cu) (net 17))
 (segment (start 133.625 58.575) (end 135.39 56.81) (width 0.25) (layer F.Cu) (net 17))
 (segment (start 134.225 46.725) (end 133.625 46.125) (width 0.25) (layer B.Cu) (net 15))
 (segment (start 136.825001 50.475001) (end 136.825001 50.299999) (width 0.25) (layer B.Cu) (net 15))
 (segment (start 136.825001 50.299999) (end 136.8 50.274998) (width 0.25) (layer B.Cu) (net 15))
 (segment (start 138.08 51.73) (end 136.825001 50.475001) (width 0.25) (layer B.Cu) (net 15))
 (segment (start 136.8 50.274998) (end 136.8 48.075) (width 0.25) (layer B.Cu) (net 15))
 (segment (start 133.625 46.125) (end 133.625 44.9) (width 0.25) (layer B.Cu) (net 15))
 (segment (start 135.45 46.725) (end 134.225 46.725) (width 0.25) (layer B.Cu) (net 15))
 (segment (start 136.8 48.075) (end 135.45 46.725) (width 0.25) (layer B.Cu) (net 15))
 (segment (start 132.375 45.95) (end 132.375 44.9) (width 0.25) (layer F.Cu) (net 18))
 (segment (start 132 46.325) (end 132.375 45.95) (width 0.25) (layer F.Cu) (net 18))
 (segment (start 129.1 46.325) (end 132 46.325) (width 0.25) (layer F.Cu) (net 18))
 (segment (start 127.92 49.19) (end 127.92 47.505) (width 0.25) (layer F.Cu) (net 18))
 (segment (start 127.92 47.505) (end 129.1 46.325) (width 0.25) (layer F.Cu) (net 18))
 (segment (start 137.13 53.32) (end 138.08 54.27) (width 0.25) (layer B.Cu) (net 10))
 (segment (start 136 53.32) (end 137.13 53.32) (width 0.25) (layer B.Cu) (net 10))
 (segment (start 131.75 61.1) (end 131.75 59.25) (width 0.25) (layer B.Cu) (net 9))
 (segment (start 131.75 59.25) (end 132.5 58.5) (width 0.25) (layer B.Cu) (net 9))
 (segment (start 132.375 58.625) (end 132.5 58.5) (width 0.25) (layer B.Cu) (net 9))
 (segment (start 130.82 53.32) (end 130 53.32) (width 0.25) (layer B.Cu) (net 9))
 (segment (start 132.5 58.5) (end 132.5 55) (width 0.25) (layer B.Cu) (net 9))
 (segment (start 132.5 55) (end 130.82 53.32) (width 0.25) (layer B.Cu) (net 9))
 (segment (start 130.93 52.68) (end 130 52.68) (width 0.25) (layer B.Cu) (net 7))
 (segment (start 133 61.1) (end 133 54.75) (width 0.25) (layer B.Cu) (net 7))
 (segment (start 133 54.75) (end 130.93 52.68) (width 0.25) (layer B.Cu) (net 7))
 (segment (start 140 53) (end 140.75 53.75) (width 0.25) (layer B.Cu) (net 8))
 (segment (start 140.75 53.75) (end 140.75 54.65) (width 0.25) (layer B.Cu) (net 8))
 (segment (start 137.446411 53) (end 140 53) (width 0.25) (layer B.Cu) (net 8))
 (segment (start 137.126411 52.68) (end 137.446411 53) (width 0.25) (layer B.Cu) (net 8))
 (segment (start 136 52.68) (end 137.126411 52.68) (width 0.25) (layer B.Cu) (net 8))
 (segment (start 132.375 44.9) (end 132.375 43.499998) (width 0.25) (layer B.Cu) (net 1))
 (segment (start 132.375 43.499998) (end 133.449998 43.499998) (width 0.25) (layer F.Cu) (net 1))
 (segment (start 133.625 43.675) (end 133.625 44.9) (width 0.25) (layer F.Cu) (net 1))
 (segment (start 133.449998 43.499998) (end 133.625 43.675) (width 0.25) (layer F.Cu) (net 1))
 (segment (start 132.375 47.15) (end 132.375 44.9) (width 0.25) (layer B.Cu) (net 1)))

